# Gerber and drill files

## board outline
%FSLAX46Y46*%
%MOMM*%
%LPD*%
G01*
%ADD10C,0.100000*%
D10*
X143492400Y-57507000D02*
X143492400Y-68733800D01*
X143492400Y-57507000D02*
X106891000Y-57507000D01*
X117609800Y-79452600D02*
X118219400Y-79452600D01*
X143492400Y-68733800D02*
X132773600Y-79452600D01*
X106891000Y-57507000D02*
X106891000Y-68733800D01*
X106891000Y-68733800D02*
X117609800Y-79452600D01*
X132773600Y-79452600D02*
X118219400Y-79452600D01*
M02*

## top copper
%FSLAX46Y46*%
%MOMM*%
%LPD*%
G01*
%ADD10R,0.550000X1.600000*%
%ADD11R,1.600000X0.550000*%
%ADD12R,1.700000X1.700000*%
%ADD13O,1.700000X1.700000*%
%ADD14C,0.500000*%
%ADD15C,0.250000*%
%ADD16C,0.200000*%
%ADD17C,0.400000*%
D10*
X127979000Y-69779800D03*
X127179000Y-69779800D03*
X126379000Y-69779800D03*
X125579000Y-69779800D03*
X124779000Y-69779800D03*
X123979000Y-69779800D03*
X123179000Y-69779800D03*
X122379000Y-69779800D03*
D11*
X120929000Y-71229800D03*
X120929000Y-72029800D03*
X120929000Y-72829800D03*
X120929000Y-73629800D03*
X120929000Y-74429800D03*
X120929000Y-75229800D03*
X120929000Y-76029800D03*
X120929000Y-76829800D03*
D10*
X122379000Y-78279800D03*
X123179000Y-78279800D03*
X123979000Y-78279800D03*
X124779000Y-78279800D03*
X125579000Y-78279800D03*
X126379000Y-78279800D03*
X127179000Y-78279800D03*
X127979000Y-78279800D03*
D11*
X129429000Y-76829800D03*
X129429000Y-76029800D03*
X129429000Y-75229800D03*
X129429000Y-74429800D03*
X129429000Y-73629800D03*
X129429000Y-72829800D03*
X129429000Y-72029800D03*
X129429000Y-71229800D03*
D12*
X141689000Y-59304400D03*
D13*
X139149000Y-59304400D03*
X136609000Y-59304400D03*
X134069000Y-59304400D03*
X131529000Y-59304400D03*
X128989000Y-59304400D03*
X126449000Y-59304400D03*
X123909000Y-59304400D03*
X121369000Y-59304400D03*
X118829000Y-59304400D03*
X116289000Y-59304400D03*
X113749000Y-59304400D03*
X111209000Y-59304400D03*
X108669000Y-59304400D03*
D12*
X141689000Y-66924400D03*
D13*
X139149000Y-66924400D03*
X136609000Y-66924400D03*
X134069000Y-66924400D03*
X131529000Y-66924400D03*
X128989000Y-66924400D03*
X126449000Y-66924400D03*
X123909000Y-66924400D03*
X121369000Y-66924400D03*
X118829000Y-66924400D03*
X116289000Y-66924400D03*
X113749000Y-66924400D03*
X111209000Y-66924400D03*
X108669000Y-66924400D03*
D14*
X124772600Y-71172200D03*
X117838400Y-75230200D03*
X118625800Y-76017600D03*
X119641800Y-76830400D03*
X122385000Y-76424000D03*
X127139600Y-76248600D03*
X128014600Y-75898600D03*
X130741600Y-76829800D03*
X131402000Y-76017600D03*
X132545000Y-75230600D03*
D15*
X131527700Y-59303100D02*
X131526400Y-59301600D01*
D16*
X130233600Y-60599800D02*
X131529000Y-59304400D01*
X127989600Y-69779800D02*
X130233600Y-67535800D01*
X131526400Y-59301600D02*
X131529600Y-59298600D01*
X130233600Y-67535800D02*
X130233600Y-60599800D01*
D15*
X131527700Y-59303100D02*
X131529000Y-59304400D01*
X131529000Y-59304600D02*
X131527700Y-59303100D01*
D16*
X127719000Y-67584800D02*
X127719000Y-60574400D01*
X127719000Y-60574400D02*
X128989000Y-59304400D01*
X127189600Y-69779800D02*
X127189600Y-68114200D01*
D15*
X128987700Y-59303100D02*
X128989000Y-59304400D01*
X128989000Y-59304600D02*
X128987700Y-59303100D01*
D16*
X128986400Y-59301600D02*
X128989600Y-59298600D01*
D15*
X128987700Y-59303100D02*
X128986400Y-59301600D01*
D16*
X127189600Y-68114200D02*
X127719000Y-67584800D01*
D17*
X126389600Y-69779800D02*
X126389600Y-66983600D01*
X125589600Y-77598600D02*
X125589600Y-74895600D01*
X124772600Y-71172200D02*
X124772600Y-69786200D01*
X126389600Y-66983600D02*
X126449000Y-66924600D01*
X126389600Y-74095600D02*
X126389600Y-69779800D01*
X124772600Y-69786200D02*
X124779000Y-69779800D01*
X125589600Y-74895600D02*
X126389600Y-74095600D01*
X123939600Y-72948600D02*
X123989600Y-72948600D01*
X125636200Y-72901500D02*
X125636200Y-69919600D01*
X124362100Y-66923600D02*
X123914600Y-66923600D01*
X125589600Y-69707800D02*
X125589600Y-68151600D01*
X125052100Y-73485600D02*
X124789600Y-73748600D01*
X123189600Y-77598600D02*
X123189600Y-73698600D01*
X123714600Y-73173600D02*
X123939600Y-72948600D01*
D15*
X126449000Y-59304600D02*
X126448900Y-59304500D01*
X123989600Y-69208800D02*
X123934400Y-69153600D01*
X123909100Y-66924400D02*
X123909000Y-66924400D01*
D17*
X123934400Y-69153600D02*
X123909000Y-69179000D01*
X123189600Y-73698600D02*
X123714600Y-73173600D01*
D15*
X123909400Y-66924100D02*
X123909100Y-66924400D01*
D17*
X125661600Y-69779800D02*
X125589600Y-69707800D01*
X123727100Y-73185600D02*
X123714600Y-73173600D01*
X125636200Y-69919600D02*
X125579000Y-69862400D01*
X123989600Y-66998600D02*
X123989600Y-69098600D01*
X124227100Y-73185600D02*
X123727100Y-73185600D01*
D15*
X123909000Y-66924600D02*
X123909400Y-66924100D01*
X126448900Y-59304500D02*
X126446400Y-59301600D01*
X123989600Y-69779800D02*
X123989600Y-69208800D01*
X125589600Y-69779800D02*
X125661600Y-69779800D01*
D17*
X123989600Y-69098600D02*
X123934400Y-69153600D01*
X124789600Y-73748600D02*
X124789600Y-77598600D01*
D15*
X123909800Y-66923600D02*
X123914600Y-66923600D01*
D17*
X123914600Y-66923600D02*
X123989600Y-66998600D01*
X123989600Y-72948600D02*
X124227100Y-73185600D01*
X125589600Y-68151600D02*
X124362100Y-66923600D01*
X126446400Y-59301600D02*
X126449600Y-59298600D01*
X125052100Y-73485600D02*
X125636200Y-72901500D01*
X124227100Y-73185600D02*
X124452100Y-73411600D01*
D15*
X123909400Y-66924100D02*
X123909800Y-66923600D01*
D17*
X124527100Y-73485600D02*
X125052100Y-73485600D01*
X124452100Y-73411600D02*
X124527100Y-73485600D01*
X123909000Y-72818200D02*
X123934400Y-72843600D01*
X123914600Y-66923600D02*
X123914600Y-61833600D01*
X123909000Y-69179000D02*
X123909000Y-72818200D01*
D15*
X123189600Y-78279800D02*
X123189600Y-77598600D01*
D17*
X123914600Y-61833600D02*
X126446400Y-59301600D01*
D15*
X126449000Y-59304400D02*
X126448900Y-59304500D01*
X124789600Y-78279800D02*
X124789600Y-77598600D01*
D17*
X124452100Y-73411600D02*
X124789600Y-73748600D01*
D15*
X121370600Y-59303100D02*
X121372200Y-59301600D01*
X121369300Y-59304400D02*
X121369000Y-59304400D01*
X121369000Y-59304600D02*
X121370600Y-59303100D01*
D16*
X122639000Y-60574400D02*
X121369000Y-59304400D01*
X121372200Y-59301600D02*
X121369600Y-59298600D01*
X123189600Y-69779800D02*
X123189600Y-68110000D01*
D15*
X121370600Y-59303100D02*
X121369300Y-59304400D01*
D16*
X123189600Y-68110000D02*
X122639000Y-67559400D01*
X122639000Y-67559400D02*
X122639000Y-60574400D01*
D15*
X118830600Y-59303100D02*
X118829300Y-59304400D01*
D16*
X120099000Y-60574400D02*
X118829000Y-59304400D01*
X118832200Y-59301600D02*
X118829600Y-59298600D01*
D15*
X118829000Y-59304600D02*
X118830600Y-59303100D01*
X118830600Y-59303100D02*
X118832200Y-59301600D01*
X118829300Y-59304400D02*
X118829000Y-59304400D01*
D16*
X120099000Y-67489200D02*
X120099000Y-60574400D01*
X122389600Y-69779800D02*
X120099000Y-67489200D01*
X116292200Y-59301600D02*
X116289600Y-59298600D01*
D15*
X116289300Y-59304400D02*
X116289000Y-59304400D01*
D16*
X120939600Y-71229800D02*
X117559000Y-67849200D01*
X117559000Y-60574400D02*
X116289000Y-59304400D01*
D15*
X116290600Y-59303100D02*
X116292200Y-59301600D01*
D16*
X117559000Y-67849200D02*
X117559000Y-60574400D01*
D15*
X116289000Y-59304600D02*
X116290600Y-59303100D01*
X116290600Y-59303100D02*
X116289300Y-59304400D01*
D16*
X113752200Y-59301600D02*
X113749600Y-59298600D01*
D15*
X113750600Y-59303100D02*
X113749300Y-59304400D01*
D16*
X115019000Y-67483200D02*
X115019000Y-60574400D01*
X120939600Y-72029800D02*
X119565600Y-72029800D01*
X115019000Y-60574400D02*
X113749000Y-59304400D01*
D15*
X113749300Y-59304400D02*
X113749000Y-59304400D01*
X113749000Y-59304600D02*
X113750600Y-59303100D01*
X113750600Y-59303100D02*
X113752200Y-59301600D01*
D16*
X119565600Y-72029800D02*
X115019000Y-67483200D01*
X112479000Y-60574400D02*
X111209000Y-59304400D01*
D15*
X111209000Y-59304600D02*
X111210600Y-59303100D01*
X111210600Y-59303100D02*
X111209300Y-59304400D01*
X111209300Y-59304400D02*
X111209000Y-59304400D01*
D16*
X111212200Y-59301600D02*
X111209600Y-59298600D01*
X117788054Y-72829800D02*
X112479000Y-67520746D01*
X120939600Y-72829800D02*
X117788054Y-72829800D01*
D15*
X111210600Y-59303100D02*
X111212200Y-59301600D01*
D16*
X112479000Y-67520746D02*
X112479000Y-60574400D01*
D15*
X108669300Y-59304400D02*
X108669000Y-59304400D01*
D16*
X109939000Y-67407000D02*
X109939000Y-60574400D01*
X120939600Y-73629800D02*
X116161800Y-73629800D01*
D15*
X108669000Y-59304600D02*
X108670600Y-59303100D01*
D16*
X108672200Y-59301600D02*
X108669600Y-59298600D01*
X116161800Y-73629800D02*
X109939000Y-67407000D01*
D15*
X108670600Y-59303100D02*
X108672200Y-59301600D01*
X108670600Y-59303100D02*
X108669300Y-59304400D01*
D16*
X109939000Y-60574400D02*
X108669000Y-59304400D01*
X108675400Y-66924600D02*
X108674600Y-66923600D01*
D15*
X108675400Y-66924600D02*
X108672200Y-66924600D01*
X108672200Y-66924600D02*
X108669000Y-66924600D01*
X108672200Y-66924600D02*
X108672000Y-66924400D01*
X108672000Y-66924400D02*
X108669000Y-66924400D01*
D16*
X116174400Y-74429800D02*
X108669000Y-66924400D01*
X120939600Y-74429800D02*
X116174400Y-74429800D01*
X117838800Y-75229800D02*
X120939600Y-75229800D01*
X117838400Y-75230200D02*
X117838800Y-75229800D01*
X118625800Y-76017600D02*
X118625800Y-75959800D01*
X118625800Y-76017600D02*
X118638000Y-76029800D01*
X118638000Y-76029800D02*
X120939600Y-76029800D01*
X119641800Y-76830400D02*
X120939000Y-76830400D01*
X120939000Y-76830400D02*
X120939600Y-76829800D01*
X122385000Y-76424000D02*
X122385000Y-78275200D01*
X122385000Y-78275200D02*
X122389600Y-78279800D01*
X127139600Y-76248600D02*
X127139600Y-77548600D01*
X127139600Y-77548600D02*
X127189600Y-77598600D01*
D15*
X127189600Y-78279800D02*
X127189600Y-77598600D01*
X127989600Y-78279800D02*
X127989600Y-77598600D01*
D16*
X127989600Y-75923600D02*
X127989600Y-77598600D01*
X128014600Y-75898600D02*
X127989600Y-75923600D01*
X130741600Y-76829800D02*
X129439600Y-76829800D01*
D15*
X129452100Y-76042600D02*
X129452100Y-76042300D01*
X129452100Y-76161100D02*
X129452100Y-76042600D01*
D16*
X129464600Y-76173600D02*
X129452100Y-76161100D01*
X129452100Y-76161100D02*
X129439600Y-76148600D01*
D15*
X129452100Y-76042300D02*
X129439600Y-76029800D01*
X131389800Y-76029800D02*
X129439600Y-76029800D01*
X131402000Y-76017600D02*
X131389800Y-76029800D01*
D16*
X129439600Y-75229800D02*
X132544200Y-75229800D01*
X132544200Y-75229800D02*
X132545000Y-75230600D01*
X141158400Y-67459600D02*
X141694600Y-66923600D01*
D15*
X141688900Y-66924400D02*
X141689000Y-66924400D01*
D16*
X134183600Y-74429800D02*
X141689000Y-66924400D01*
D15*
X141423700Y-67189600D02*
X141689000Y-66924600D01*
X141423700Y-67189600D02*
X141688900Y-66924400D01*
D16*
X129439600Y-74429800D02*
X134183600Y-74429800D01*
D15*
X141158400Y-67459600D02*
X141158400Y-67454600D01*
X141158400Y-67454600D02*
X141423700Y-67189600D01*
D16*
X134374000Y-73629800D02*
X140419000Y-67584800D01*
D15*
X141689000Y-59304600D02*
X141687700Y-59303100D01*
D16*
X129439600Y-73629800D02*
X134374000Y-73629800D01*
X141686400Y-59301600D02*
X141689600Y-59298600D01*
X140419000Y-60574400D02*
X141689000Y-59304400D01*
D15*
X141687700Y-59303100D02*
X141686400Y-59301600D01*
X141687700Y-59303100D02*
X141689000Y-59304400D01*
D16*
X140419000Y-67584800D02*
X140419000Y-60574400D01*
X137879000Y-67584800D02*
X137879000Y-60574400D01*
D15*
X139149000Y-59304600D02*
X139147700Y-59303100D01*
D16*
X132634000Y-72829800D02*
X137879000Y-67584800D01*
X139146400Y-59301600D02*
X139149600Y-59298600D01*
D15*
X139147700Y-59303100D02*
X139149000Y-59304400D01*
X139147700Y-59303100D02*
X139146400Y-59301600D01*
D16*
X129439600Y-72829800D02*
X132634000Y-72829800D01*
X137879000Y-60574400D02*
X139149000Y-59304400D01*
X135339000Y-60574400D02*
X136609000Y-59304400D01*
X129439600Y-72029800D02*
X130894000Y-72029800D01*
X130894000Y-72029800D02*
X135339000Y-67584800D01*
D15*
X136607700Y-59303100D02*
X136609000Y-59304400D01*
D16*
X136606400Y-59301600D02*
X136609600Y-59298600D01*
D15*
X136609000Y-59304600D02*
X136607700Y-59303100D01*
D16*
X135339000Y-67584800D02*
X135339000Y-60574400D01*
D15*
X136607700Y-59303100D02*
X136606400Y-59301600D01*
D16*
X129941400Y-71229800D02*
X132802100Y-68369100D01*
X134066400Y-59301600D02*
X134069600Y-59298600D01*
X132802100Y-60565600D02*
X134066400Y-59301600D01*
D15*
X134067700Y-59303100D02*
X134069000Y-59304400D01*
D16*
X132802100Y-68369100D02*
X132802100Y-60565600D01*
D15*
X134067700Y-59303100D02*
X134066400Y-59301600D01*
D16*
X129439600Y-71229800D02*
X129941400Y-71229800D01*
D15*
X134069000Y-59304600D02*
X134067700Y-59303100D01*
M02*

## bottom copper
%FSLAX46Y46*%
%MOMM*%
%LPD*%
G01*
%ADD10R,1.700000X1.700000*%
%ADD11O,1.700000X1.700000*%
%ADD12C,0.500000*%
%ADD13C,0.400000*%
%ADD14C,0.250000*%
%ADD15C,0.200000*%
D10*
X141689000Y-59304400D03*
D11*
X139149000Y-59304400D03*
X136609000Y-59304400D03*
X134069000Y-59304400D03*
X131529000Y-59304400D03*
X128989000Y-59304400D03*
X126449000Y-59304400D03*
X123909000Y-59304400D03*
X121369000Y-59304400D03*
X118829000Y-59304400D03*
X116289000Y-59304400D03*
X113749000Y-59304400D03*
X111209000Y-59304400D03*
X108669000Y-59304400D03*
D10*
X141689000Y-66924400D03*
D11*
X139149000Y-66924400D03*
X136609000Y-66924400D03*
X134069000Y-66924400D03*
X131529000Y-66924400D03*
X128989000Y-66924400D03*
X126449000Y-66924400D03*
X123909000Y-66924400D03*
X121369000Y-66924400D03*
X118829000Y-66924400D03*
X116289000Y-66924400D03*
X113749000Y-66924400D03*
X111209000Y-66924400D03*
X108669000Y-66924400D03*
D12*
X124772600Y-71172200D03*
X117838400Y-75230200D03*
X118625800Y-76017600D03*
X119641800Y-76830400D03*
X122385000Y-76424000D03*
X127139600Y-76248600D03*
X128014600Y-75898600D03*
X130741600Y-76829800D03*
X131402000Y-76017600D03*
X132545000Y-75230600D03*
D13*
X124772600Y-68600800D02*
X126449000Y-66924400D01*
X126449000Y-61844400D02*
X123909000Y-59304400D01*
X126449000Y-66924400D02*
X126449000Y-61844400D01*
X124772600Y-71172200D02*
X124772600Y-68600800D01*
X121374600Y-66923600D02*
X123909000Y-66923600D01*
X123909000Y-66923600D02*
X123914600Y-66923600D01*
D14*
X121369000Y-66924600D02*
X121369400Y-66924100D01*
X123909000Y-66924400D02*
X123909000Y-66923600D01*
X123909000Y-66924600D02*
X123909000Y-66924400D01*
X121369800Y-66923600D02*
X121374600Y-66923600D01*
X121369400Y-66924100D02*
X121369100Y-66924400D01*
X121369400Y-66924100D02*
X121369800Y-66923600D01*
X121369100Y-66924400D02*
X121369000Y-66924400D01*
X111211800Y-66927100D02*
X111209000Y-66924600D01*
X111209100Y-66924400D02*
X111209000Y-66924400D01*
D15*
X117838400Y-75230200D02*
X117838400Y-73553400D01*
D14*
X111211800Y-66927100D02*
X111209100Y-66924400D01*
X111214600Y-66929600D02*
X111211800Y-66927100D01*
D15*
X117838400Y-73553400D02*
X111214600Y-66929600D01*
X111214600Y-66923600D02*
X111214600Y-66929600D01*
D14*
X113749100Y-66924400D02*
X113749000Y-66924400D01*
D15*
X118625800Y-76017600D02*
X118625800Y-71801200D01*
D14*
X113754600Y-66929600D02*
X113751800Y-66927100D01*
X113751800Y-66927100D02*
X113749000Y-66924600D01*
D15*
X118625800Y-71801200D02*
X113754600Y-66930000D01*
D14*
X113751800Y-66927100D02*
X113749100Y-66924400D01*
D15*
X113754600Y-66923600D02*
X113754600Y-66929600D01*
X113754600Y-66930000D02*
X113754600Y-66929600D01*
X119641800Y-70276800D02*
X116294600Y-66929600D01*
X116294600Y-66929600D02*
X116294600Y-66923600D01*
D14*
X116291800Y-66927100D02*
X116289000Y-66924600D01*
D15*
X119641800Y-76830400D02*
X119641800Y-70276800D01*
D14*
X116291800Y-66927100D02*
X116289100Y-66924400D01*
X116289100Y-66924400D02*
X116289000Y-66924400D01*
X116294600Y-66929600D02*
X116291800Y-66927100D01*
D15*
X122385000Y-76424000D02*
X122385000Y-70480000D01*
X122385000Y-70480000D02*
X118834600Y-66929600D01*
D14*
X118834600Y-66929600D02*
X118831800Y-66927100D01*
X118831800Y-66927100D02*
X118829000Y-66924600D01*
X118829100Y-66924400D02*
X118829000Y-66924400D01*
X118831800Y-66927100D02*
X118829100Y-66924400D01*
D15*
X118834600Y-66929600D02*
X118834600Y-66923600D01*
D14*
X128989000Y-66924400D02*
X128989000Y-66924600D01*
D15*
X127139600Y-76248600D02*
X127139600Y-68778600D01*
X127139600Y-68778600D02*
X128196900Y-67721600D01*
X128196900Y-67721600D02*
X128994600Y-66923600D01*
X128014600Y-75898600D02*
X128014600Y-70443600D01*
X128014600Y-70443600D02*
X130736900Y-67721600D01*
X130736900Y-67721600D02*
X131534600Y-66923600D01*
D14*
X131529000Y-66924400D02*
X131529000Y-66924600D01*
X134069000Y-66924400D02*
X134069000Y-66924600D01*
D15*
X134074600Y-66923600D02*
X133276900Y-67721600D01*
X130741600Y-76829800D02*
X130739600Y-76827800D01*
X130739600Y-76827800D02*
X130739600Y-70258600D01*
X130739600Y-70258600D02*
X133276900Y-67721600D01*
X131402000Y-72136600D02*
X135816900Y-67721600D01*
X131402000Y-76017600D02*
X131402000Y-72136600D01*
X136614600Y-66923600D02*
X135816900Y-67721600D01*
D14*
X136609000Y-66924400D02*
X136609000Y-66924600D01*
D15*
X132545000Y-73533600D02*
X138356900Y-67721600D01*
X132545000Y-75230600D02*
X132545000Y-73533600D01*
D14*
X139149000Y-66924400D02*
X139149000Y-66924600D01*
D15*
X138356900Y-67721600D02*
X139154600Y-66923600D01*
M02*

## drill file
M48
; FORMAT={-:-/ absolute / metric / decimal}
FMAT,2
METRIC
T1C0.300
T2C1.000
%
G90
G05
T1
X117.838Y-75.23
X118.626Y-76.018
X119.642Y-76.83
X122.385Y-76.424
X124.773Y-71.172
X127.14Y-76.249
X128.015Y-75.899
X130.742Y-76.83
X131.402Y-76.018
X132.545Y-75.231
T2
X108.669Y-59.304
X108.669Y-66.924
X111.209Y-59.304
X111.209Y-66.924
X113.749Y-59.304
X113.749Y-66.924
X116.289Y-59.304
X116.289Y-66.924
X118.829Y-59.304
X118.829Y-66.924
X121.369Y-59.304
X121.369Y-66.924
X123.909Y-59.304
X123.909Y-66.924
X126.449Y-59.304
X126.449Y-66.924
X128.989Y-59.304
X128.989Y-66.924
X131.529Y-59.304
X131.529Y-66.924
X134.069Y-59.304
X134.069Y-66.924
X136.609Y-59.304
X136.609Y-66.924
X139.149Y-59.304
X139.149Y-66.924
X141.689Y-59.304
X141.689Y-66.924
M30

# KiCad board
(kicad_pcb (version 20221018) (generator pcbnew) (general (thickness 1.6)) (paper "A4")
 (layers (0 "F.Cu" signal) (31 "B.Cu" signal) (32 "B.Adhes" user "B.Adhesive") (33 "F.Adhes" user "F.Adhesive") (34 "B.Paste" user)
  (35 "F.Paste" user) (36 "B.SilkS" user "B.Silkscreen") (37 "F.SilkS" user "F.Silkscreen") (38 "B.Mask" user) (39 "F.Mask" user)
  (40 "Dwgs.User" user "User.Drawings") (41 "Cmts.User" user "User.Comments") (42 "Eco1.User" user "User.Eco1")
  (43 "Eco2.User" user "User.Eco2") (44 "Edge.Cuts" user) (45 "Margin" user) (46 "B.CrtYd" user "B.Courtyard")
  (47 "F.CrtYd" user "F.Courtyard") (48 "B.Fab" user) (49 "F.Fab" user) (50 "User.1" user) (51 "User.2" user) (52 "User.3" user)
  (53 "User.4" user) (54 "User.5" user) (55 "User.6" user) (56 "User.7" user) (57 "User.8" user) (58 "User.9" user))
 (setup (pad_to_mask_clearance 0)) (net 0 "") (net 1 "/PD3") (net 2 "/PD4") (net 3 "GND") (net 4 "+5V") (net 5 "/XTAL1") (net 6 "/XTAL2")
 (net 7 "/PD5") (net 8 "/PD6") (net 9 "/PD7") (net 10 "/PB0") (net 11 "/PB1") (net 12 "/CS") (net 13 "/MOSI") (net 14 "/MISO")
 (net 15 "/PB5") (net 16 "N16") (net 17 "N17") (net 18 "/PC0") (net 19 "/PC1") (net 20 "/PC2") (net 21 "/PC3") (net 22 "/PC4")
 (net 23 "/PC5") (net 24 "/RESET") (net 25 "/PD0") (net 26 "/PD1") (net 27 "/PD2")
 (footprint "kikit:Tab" (layer "F.Cu") (at 113.0505 57.277 -90)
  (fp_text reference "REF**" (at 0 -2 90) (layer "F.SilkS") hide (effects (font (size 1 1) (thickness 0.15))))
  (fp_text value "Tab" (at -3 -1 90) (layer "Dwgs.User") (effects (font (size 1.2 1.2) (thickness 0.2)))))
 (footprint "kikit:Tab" (layer "F.Cu") (at 125.4965 79.7052 90)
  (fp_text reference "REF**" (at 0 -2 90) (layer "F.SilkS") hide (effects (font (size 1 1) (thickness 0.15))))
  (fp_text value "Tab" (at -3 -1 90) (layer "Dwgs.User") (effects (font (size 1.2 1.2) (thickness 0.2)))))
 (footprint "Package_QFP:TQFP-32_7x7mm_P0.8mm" (layer "F.Cu") (at 125.179 74.0298 -90)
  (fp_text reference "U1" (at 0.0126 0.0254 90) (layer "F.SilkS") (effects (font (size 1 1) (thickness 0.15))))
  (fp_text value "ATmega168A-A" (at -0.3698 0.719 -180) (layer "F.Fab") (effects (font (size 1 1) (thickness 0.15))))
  (pad "1" smd rect (at -4.25 -2.8 270) (size 1.6 0.55) (layers "F.Cu" "F.Paste" "F.Mask") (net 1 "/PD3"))
  (pad "2" smd rect (at -4.25 -2 270) (size 1.6 0.55) (layers "F.Cu" "F.Paste" "F.Mask") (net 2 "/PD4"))
  (pad "3" smd rect (at -4.25 -1.2 270) (size 1.6 0.55) (layers "F.Cu" "F.Paste" "F.Mask") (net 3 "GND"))
  (pad "4" smd rect (at -4.25 -0.4 270) (size 1.6 0.55) (layers "F.Cu" "F.Paste" "F.Mask") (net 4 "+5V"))
  (pad "5" smd rect (at -4.25 0.4 270) (size 1.6 0.55) (layers "F.Cu" "F.Paste" "F.Mask") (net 3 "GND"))
  (pad "6" smd rect (at -4.25 1.2 270) (size 1.6 0.55) (layers "F.Cu" "F.Paste" "F.Mask") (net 4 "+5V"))
  (pad "7" smd rect (at -4.25 2 270) (size 1.6 0.55) (layers "F.Cu" "F.Paste" "F.Mask") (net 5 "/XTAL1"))
  (pad "8" smd rect (at -4.25 2.8 270) (size 1.6 0.55) (layers "F.Cu" "F.Paste" "F.Mask") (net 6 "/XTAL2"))
  (pad "9" smd rect (at -2.8 4.25) (size 1.6 0.55) (layers "F.Cu" "F.Paste" "F.Mask") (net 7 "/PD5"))
  (pad "10" smd rect (at -2 4.25) (size 1.6 0.55) (layers "F.Cu" "F.Paste" "F.Mask") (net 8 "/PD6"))
  (pad "11" smd rect (at -1.2 4.25) (size 1.6 0.55) (layers "F.Cu" "F.Paste" "F.Mask") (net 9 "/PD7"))
  (pad "12" smd rect (at -0.4 4.25) (size 1.6 0.55) (layers "F.Cu" "F.Paste" "F.Mask") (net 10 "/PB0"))
  (pad "13" smd rect (at 0.4 4.25) (size 1.6 0.55) (layers "F.Cu" "F.Paste" "F.Mask") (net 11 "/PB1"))
  (pad "14" smd rect (at 1.2 4.25) (size 1.6 0.55) (layers "F.Cu" "F.Paste" "F.Mask") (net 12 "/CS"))
  (pad "15" smd rect (at 2 4.25) (size 1.6 0.55) (layers "F.Cu" "F.Paste" "F.Mask") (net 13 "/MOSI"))
  (pad "16" smd rect (at 2.8 4.25) (size 1.6 0.55) (layers "F.Cu" "F.Paste" "F.Mask") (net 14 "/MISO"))
  (pad "17" smd rect (at 4.25 2.8 270) (size 1.6 0.55) (layers "F.Cu" "F.Paste" "F.Mask") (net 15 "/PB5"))
  (pad "18" smd rect (at 4.25 2 270) (size 1.6 0.55) (layers "F.Cu" "F.Paste" "F.Mask") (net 4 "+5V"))
  (pad "19" smd rect (at 4.25 1.2 270) (size 1.6 0.55) (layers "F.Cu" "F.Paste" "F.Mask") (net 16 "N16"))
  (pad "20" smd rect (at 4.25 0.4 270) (size 1.6 0.55) (layers "F.Cu" "F.Paste" "F.Mask") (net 4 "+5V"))
  (pad "21" smd rect (at 4.25 -0.4 270) (size 1.6 0.55) (layers "F.Cu" "F.Paste" "F.Mask") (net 3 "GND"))
  (pad "22" smd rect (at 4.25 -1.2 270) (size 1.6 0.55) (layers "F.Cu" "F.Paste" "F.Mask") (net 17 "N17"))
  (pad "23" smd rect (at 4.25 -2 270) (size 1.6 0.55) (layers "F.Cu" "F.Paste" "F.Mask") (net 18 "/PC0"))
  (pad "24" smd rect (at 4.25 -2.8 270) (size 1.6 0.55) (layers "F.Cu" "F.Paste" "F.Mask") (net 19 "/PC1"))
  (pad "25" smd rect (at 2.8 -4.25) (size 1.6 0.55) (layers "F.Cu" "F.Paste" "F.Mask") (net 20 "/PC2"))
  (pad "26" smd rect (at 2 -4.25) (size 1.6 0.55) (layers "F.Cu" "F.Paste" "F.Mask") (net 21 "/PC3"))
  (pad "27" smd rect (at 1.2 -4.25) (size 1.6 0.55) (layers "F.Cu" "F.Paste" "F.Mask") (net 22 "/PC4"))
  (pad "28" smd rect (at 0.4 -4.25) (size 1.6 0.55) (layers "F.Cu" "F.Paste" "F.Mask") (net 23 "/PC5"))
  (pad "29" smd rect (at -0.4 -4.25) (size 1.6 0.55) (layers "F.Cu" "F.Paste" "F.Mask") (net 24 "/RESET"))
  (pad "30" smd rect (at -1.2 -4.25) (size 1.6 0.55) (layers "F.Cu" "F.Paste" "F.Mask") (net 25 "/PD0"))
  (pad "31" smd rect (at -2 -4.25) (size 1.6 0.55) (layers "F.Cu" "F.Paste" "F.Mask") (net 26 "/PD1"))
  (pad "32" smd rect (at -2.8 -4.25) (size 1.6 0.55) (layers "F.Cu" "F.Paste" "F.Mask") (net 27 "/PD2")))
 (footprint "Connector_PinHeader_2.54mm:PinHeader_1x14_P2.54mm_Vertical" (layer "F.Cu") (at 141.689 59.3044 -90)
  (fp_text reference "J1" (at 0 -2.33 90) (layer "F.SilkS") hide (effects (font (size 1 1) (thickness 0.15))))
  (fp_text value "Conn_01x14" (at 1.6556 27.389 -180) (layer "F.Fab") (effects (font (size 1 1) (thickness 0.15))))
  (pad "1" thru_hole rect (at 0 0 270) (size 1.7 1.7) (drill 1) (layers "*.Cu" "*.Mask") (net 24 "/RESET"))
  (pad "2" thru_hole oval (at 0 2.54 270) (size 1.7 1.7) (drill 1) (layers "*.Cu" "*.Mask") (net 25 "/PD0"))
  (pad "3" thru_hole oval (at 0 5.08 270) (size 1.7 1.7) (drill 1) (layers "*.Cu" "*.Mask") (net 26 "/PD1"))
  (pad "4" thru_hole oval (at 0 7.62 270) (size 1.7 1.7) (drill 1) (layers "*.Cu" "*.Mask") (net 27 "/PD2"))
  (pad "5" thru_hole oval (at 0 10.16 270) (size 1.7 1.7) (drill 1) (layers "*.Cu" "*.Mask") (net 1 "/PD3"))
  (pad "6" thru_hole oval (at 0 12.7 270) (size 1.7 1.7) (drill 1) (layers "*.Cu" "*.Mask") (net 2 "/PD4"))
  (pad "7" thru_hole oval (at 0 15.24 270) (size 1.7 1.7) (drill 1) (layers "*.Cu" "*.Mask") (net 4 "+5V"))
  (pad "8" thru_hole oval (at 0 17.78 270) (size 1.7 1.7) (drill 1) (layers "*.Cu" "*.Mask") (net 3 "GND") (zone_connect 2))
  (pad "9" thru_hole oval (at 0 20.32 270) (size 1.7 1.7) (drill 1) (layers "*.Cu" "*.Mask") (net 5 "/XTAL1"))
  (pad "10" thru_hole oval (at 0 22.86 270) (size 1.7 1.7) (drill 1) (layers "*.Cu" "*.Mask") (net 6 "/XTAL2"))
  (pad "11" thru_hole oval (at 0 25.4 270) (size 1.7 1.7) (drill 1) (layers "*.Cu" "*.Mask") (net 7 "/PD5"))
  (pad "12" thru_hole oval (at 0 27.94 270) (size 1.7 1.7) (drill 1) (layers "*.Cu" "*.Mask") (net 8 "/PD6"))
  (pad "13" thru_hole oval (at 0 30.48 270) (size 1.7 1.7) (drill 1) (layers "*.Cu" "*.Mask") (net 9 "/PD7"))
  (pad "14" thru_hole oval (at 0 33.02 270) (size 1.7 1.7) (drill 1) (layers "*.Cu" "*.Mask") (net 10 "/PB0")))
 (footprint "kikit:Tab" (layer "F.Cu") (at 143.7386 63.1204 180)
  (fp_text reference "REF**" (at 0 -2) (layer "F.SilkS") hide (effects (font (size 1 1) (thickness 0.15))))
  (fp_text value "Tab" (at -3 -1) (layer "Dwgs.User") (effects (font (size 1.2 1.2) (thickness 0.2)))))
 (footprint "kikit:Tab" (layer "F.Cu") (at 137.3329 57.2262 -90)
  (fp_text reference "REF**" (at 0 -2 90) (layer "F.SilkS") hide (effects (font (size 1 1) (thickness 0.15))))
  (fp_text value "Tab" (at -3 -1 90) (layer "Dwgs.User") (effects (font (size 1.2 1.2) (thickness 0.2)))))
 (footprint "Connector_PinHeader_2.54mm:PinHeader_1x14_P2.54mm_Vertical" (layer "F.Cu") (at 141.689 66.9244 -90)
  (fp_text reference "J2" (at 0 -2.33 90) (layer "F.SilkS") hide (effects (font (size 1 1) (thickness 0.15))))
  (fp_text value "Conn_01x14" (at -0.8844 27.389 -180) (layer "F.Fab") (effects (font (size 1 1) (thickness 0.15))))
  (pad "1" thru_hole rect (at 0 0 270) (size 1.7 1.7) (drill 1) (layers "*.Cu" "*.Mask") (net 23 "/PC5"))
  (pad "2" thru_hole oval (at 0 2.54 270) (size 1.7 1.7) (drill 1) (layers "*.Cu" "*.Mask") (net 22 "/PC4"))
  (pad "3" thru_hole oval (at 0 5.08 270) (size 1.7 1.7) (drill 1) (layers "*.Cu" "*.Mask") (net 21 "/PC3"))
  (pad "4" thru_hole oval (at 0 7.62 270) (size 1.7 1.7) (drill 1) (layers "*.Cu" "*.Mask") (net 20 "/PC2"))
  (pad "5" thru_hole oval (at 0 10.16 270) (size 1.7 1.7) (drill 1) (layers "*.Cu" "*.Mask") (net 19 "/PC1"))
  (pad "6" thru_hole oval (at 0 12.7 270) (size 1.7 1.7) (drill 1) (layers "*.Cu" "*.Mask") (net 18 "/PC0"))
  (pad "7" thru_hole oval (at 0 15.24 270) (size 1.7 1.7) (drill 1) (layers "*.Cu" "*.Mask") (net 3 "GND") (zone_connect 2))
  (pad "8" thru_hole oval (at 0 17.78 270) (size 1.7 1.7) (drill 1) (layers "*.Cu" "*.Mask") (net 4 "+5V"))
  (pad "9" thru_hole oval (at 0 20.32 270) (size 1.7 1.7) (drill 1) (layers "*.Cu" "*.Mask") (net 4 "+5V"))
  (pad "10" thru_hole oval (at 0 22.86 270) (size 1.7 1.7) (drill 1) (layers "*.Cu" "*.Mask") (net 15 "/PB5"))
  (pad "11" thru_hole oval (at 0 25.4 270) (size 1.7 1.7) (drill 1) (layers "*.Cu" "*.Mask") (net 14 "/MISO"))
  (pad "12" thru_hole oval (at 0 27.94 270) (size 1.7 1.7) (drill 1) (layers "*.Cu" "*.Mask") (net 13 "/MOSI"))
  (pad "13" thru_hole oval (at 0 30.48 270) (size 1.7 1.7) (drill 1) (layers "*.Cu" "*.Mask") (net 12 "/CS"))
  (pad "14" thru_hole oval (at 0 33.02 270) (size 1.7 1.7) (drill 1) (layers "*.Cu" "*.Mask") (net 11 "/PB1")))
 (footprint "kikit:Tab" (layer "F.Cu") (at 106.6292 63.1204)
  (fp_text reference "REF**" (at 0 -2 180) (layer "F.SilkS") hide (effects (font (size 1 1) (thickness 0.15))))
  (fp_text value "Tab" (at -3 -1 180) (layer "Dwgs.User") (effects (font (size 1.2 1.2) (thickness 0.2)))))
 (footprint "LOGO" (layer "B.Cu") (at 125.179 74.0298 180)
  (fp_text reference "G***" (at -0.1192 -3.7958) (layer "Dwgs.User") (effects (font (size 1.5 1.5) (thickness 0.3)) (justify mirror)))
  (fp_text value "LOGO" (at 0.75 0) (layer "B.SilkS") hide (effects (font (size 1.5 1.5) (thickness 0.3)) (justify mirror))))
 (gr_line (start 143.4924 57.507) (end 143.4924 68.7338) (stroke (width 0.1) (type default)) (layer "Edge.Cuts"))
 (gr_line (start 143.4924 57.507) (end 106.891 57.507) (stroke (width 0.1) (type default)) (layer "Edge.Cuts"))
 (gr_line (start 117.6098 79.4526) (end 118.2194 79.4526) (stroke (width 0.1) (type default)) (layer "Edge.Cuts"))
 (gr_line (start 143.4924 68.7338) (end 132.7736 79.4526) (stroke (width 0.1) (type default)) (layer "Edge.Cuts"))
 (gr_line (start 106.891 57.507) (end 106.891 68.7338) (stroke (width 0.1) (type default)) (layer "Edge.Cuts"))
 (gr_line (start 106.891 68.7338) (end 117.6098 79.4526) (stroke (width 0.1) (type default)) (layer "Edge.Cuts"))
 (gr_line (start 132.7736 79.4526) (end 118.2194 79.4526) (stroke (width 0.1) (type default)) (layer "Edge.Cuts"))
 (segment (start 131.5277 59.3031) (end 131.5264 59.3016) (width 0.25) (layer "F.Cu") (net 1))
 (segment (start 130.2336 60.5998) (end 131.529 59.3044) (width 0.2) (layer "F.Cu") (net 1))
 (segment (start 127.9896 69.7798) (end 130.2336 67.5358) (width 0.2) (layer "F.Cu") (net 1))
 (segment (start 131.5264 59.3016) (end 131.5296 59.2986) (width 0.2) (layer "F.Cu") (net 1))
 (segment (start 130.2336 67.5358) (end 130.2336 60.5998) (width 0.2) (layer "F.Cu") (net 1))
 (segment (start 131.5277 59.3031) (end 131.529 59.3044) (width 0.25) (layer "F.Cu") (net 1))
 (segment (start 131.529 59.3046) (end 131.5277 59.3031) (width 0.25) (layer "F.Cu") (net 1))
 (segment (start 127.719 67.5848) (end 127.719 60.5744) (width 0.2) (layer "F.Cu") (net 2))
 (segment (start 127.719 60.5744) (end 128.989 59.3044) (width 0.2) (layer "F.Cu") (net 2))
 (segment (start 127.1896 69.7798) (end 127.1896 68.1142) (width 0.2) (layer "F.Cu") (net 2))
 (segment (start 128.9877 59.3031) (end 128.989 59.3044) (width 0.25) (layer "F.Cu") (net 2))
 (segment (start 128.989 59.3046) (end 128.9877 59.3031) (width 0.25) (layer "F.Cu") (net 2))
 (segment (start 128.9864 59.3016) (end 128.9896 59.2986) (width 0.2) (layer "F.Cu") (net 2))
 (segment (start 128.9877 59.3031) (end 128.9864 59.3016) (width 0.25) (layer "F.Cu") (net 2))
 (segment (start 127.1896 68.1142) (end 127.719 67.5848) (width 0.2) (layer "F.Cu") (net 2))
 (segment (start 126.3896 69.7798) (end 126.3896 66.9836) (width 0.4) (layer "F.Cu") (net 3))
 (segment (start 125.5896 77.5986) (end 125.5896 74.8956) (width 0.4) (layer "F.Cu") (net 3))
 (segment (start 124.7726 71.1722) (end 124.7726 69.7862) (width 0.4) (layer "F.Cu") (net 3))
 (segment (start 126.3896 66.9836) (end 126.449 66.9246) (width 0.4) (layer "F.Cu") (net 3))
 (segment (start 126.3896 74.0956) (end 126.3896 69.7798) (width 0.4) (layer "F.Cu") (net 3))
 (segment (start 124.7726 69.7862) (end 124.779 69.7798) (width 0.4) (layer "F.Cu") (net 3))
 (segment (start 125.5896 74.8956) (end 126.3896 74.0956) (width 0.4) (layer "F.Cu") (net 3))
 (via (at 124.7726 71.1722) (size 0.5) (drill 0.3) (layers "F.Cu" "B.Cu") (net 3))
 (segment (start 124.7726 68.6008) (end 126.449 66.9244) (width 0.4) (layer "B.Cu") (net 3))
 (segment (start 126.449 61.8444) (end 123.909 59.3044) (width 0.4) (layer "B.Cu") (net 3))
 (segment (start 126.449 66.9244) (end 126.449 61.8444) (width 0.4) (layer "B.Cu") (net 3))
 (segment (start 124.7726 71.1722) (end 124.7726 68.6008) (width 0.4) (layer "B.Cu") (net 3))
 (segment (start 123.9396 72.9486) (end 123.9896 72.9486) (width 0.4) (layer "F.Cu") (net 4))
 (segment (start 125.6362 72.9015) (end 125.6362 69.9196) (width 0.4) (layer "F.Cu") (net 4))
 (segment (start 124.3621 66.9236) (end 123.9146 66.9236) (width 0.4) (layer "F.Cu") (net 4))
 (segment (start 125.5896 69.7078) (end 125.5896 68.1516) (width 0.4) (layer "F.Cu") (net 4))
 (segment (start 125.0521 73.4856) (end 124.7896 73.7486) (width 0.4) (layer "F.Cu") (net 4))
 (segment (start 123.1896 77.5986) (end 123.1896 73.6986) (width 0.4) (layer "F.Cu") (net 4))
 (segment (start 123.7146 73.1736) (end 123.9396 72.9486) (width 0.4) (layer "F.Cu") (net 4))
 (segment (start 126.449 59.3046) (end 126.4489 59.3045) (width 0.25) (layer "F.Cu") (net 4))
 (segment (start 123.9896 69.2088) (end 123.9344 69.1536) (width 0.25) (layer "F.Cu") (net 4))
 (segment (start 123.9091 66.9244) (end 123.909 66.9244) (width 0.25) (layer "F.Cu") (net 4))
 (segment (start 123.9344 69.1536) (end 123.909 69.179) (width 0.4) (layer "F.Cu") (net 4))
 (segment (start 123.1896 73.6986) (end 123.7146 73.1736) (width 0.4) (layer "F.Cu") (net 4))
 (segment (start 123.9094 66.9241) (end 123.9091 66.9244) (width 0.25) (layer "F.Cu") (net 4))
 (segment (start 125.6616 69.7798) (end 125.5896 69.7078) (width 0.4) (layer "F.Cu") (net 4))
 (segment (start 123.7271 73.1856) (end 123.7146 73.1736) (width 0.4) (layer "F.Cu") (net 4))
 (segment (start 125.6362 69.9196) (end 125.579 69.8624) (width 0.4) (layer "F.Cu") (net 4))
 (segment (start 123.9896 66.9986) (end 123.9896 69.0986) (width 0.4) (layer "F.Cu") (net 4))
 (segment (start 124.2271 73.1856) (end 123.7271 73.1856) (width 0.4) (layer "F.Cu") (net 4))
 (segment (start 123.909 66.9246) (end 123.9094 66.9241) (width 0.25) (layer "F.Cu") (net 4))
 (segment (start 126.4489 59.3045) (end 126.4464 59.3016) (width 0.25) (layer "F.Cu") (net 4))
 (segment (start 123.9896 69.7798) (end 123.9896 69.2088) (width 0.25) (layer "F.Cu") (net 4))
 (segment (start 125.5896 69.7798) (end 125.6616 69.7798) (width 0.25) (layer "F.Cu") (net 4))
 (segment (start 123.9896 69.0986) (end 123.9344 69.1536) (width 0.4) (layer "F.Cu") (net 4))
 (segment (start 124.7896 73.7486) (end 124.7896 77.5986) (width 0.4) (layer "F.Cu") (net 4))
 (segment (start 123.9098 66.9236) (end 123.9146 66.9236) (width 0.25) (layer "F.Cu") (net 4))
 (segment (start 123.9146 66.9236) (end 123.9896 66.9986) (width 0.4) (layer "F.Cu") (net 4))
 (segment (start 123.9896 72.9486) (end 124.2271 73.1856) (width 0.4) (layer "F.Cu") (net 4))
 (segment (start 125.5896 68.1516) (end 124.3621 66.9236) (width 0.4) (layer "F.Cu") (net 4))
 (segment (start 126.4464 59.3016) (end 126.4496 59.2986) (width 0.4) (layer "F.Cu") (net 4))
 (segment (start 125.0521 73.4856) (end 125.6362 72.9015) (width 0.4) (layer "F.Cu") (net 4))
 (segment (start 124.2271 73.1856) (end 124.4521 73.4116) (width 0.4) (layer "F.Cu") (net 4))
 (segment (start 123.9094 66.9241) (end 123.9098 66.9236) (width 0.25) (layer "F.Cu") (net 4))
 (segment (start 124.5271 73.4856) (end 125.0521 73.4856) (width 0.4) (layer "F.Cu") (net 4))
 (segment (start 124.4521 73.4116) (end 124.5271 73.4856) (width 0.4) (layer "F.Cu") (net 4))
 (segment (start 123.909 72.8182) (end 123.9344 72.8436) (width 0.4) (layer "F.Cu") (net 4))
 (segment (start 123.9146 66.9236) (end 123.9146 61.8336) (width 0.4) (layer "F.Cu") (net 4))
 (segment (start 123.909 69.179) (end 123.909 72.8182) (width 0.4) (layer "F.Cu") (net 4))
 (segment (start 123.1896 78.2798) (end 123.1896 77.5986) (width 0.25) (layer "F.Cu") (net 4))
 (segment (start 123.9146 61.8336) (end 126.4464 59.3016) (width 0.4) (layer "F.Cu") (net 4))
 (segment (start 126.449 59.3044) (end 126.4489 59.3045) (width 0.25) (layer "F.Cu") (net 4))
 (segment (start 124.7896 78.2798) (end 124.7896 77.5986) (width 0.25) (layer "F.Cu") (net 4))
 (segment (start 124.4521 73.4116) (end 124.7896 73.7486) (width 0.4) (layer "F.Cu") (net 4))
 (segment (start 121.3746 66.9236) (end 123.909 66.9236) (width 0.4) (layer "B.Cu") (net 4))
 (segment (start 123.909 66.9236) (end 123.9146 66.9236) (width 0.4) (layer "B.Cu") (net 4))
 (segment (start 121.369 66.9246) (end 121.3694 66.9241) (width 0.25) (layer "B.Cu") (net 4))
 (segment (start 123.909 66.9244) (end 123.909 66.9236) (width 0.25) (layer "B.Cu") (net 4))
 (segment (start 123.909 66.9246) (end 123.909 66.9244) (width 0.25) (layer "B.Cu") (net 4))
 (segment (start 121.3698 66.9236) (end 121.3746 66.9236) (width 0.25) (layer "B.Cu") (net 4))
 (segment (start 121.3694 66.9241) (end 121.3691 66.9244) (width 0.25) (layer "B.Cu") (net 4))
 (segment (start 121.3694 66.9241) (end 121.3698 66.9236) (width 0.25) (layer "B.Cu") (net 4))
 (segment (start 121.3691 66.9244) (end 121.369 66.9244) (width 0.25) (layer "B.Cu") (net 4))
 (segment (start 121.3706 59.3031) (end 121.3722 59.3016) (width 0.25) (layer "F.Cu") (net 5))
 (segment (start 121.3693 59.3044) (end 121.369 59.3044) (width 0.25) (layer "F.Cu") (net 5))
 (segment (start 121.369 59.3046) (end 121.3706 59.3031) (width 0.25) (layer "F.Cu") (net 5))
 (segment (start 122.639 60.5744) (end 121.369 59.3044) (width 0.2) (layer "F.Cu") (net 5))
 (segment (start 121.3722 59.3016) (end 121.3696 59.2986) (width 0.2) (layer "F.Cu") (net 5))
 (segment (start 123.1896 69.7798) (end 123.1896 68.11) (width 0.2) (layer "F.Cu") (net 5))
 (segment (start 121.3706 59.3031) (end 121.3693 59.3044) (width 0.25) (layer "F.Cu") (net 5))
 (segment (start 123.1896 68.11) (end 122.639 67.5594) (width 0.2) (layer "F.Cu") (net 5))
 (segment (start 122.639 67.5594) (end 122.639 60.5744) (width 0.2) (layer "F.Cu") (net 5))
 (segment (start 118.8306 59.3031) (end 118.8293 59.3044) (width 0.25) (layer "F.Cu") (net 6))
 (segment (start 120.099 60.5744) (end 118.829 59.3044) (width 0.2) (layer "F.Cu") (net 6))
 (segment (start 118.8322 59.3016) (end 118.8296 59.2986) (width 0.2) (layer "F.Cu") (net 6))
 (segment (start 118.829 59.3046) (end 118.8306 59.3031) (width 0.25) (layer "F.Cu") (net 6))
 (segment (start 118.8306 59.3031) (end 118.8322 59.3016) (width 0.25) (layer "F.Cu") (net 6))
 (segment (start 118.8293 59.3044) (end 118.829 59.3044) (width 0.25) (layer "F.Cu") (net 6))
 (segment (start 120.099 67.4892) (end 120.099 60.5744) (width 0.2) (layer "F.Cu") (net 6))
 (segment (start 122.3896 69.7798) (end 120.099 67.4892) (width 0.2) (layer "F.Cu") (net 6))
 (segment (start 116.2922 59.3016) (end 116.2896 59.2986) (width 0.2) (layer "F.Cu") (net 7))
 (segment (start 116.2893 59.3044) (end 116.289 59.3044) (width 0.25) (layer "F.Cu") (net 7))
 (segment (start 120.9396 71.2298) (end 117.559 67.8492) (width 0.2) (layer "F.Cu") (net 7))
 (segment (start 117.559 60.5744) (end 116.289 59.3044) (width 0.2) (layer "F.Cu") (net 7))
 (segment (start 116.2906 59.3031) (end 116.2922 59.3016) (width 0.25) (layer "F.Cu") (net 7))
 (segment (start 117.559 67.8492) (end 117.559 60.5744) (width 0.2) (layer "F.Cu") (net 7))
 (segment (start 116.289 59.3046) (end 116.2906 59.3031) (width 0.25) (layer "F.Cu") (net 7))
 (segment (start 116.2906 59.3031) (end 116.2893 59.3044) (width 0.25) (layer "F.Cu") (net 7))
 (segment (start 113.7522 59.3016) (end 113.7496 59.2986) (width 0.2) (layer "F.Cu") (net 8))
 (segment (start 113.7506 59.3031) (end 113.7493 59.3044) (width 0.25) (layer "F.Cu") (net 8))
 (segment (start 115.019 67.4832) (end 115.019 60.5744) (width 0.2) (layer "F.Cu") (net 8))
 (segment (start 120.9396 72.0298) (end 119.5656 72.0298) (width 0.2) (layer "F.Cu") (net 8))
 (segment (start 115.019 60.5744) (end 113.749 59.3044) (width 0.2) (layer "F.Cu") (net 8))
 (segment (start 113.7493 59.3044) (end 113.749 59.3044) (width 0.25) (layer "F.Cu") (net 8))
 (segment (start 113.749 59.3046) (end 113.7506 59.3031) (width 0.25) (layer "F.Cu") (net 8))
 (segment (start 113.7506 59.3031) (end 113.7522 59.3016) (width 0.25) (layer "F.Cu") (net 8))
 (segment (start 119.5656 72.0298) (end 115.019 67.4832) (width 0.2) (layer "F.Cu") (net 8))
 (segment (start 112.479 60.5744) (end 111.209 59.3044) (width 0.2) (layer "F.Cu") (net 9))
 (segment (start 111.209 59.3046) (end 111.2106 59.3031) (width 0.25) (layer "F.Cu") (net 9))
 (segment (start 111.2106 59.3031) (end 111.2093 59.3044) (width 0.25) (layer "F.Cu") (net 9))
 (segment (start 111.2093 59.3044) (end 111.209 59.3044) (width 0.25) (layer "F.Cu") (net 9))
 (segment (start 111.2122 59.3016) (end 111.2096 59.2986) (width 0.2) (layer "F.Cu") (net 9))
 (segment (start 117.788054 72.8298) (end 112.479 67.520746) (width 0.2) (layer "F.Cu") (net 9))
 (segment (start 120.9396 72.8298) (end 117.788054 72.8298) (width 0.2) (layer "F.Cu") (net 9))
 (segment (start 111.2106 59.3031) (end 111.2122 59.3016) (width 0.25) (layer "F.Cu") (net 9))
 (segment (start 112.479 67.520746) (end 112.479 60.5744) (width 0.2) (layer "F.Cu") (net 9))
 (segment (start 108.6693 59.3044) (end 108.669 59.3044) (width 0.25) (layer "F.Cu") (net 10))
 (segment (start 109.939 67.407) (end 109.939 60.5744) (width 0.2) (layer "F.Cu") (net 10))
 (segment (start 120.9396 73.6298) (end 116.1618 73.6298) (width 0.2) (layer "F.Cu") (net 10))
 (segment (start 108.669 59.3046) (end 108.6706 59.3031) (width 0.25) (layer "F.Cu") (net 10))
 (segment (start 108.6722 59.3016) (end 108.6696 59.2986) (width 0.2) (layer "F.Cu") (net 10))
 (segment (start 116.1618 73.6298) (end 109.939 67.407) (width 0.2) (layer "F.Cu") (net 10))
 (segment (start 108.6706 59.3031) (end 108.6722 59.3016) (width 0.25) (layer "F.Cu") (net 10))
 (segment (start 108.6706 59.3031) (end 108.6693 59.3044) (width 0.25) (layer "F.Cu") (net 10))
 (segment (start 109.939 60.5744) (end 108.669 59.3044) (width 0.2) (layer "F.Cu") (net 10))
 (segment (start 108.6754 66.9246) (end 108.6746 66.9236) (width 0.2) (layer "F.Cu") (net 11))
 (segment (start 108.6754 66.9246) (end 108.6722 66.9246) (width 0.25) (layer "F.Cu") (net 11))
 (segment (start 108.6722 66.9246) (end 108.669 66.9246) (width 0.25) (layer "F.Cu") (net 11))
 (segment (start 108.6722 66.9246) (end 108.672 66.9244) (width 0.25) (layer "F.Cu") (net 11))
 (segment (start 108.672 66.9244) (end 108.669 66.9244) (width 0.25) (layer "F.Cu") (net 11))
 (segment (start 116.1744 74.4298) (end 108.669 66.9244) (width 0.2) (layer "F.Cu") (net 11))
 (segment (start 120.9396 74.4298) (end 116.1744 74.4298) (width 0.2) (layer "F.Cu") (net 11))
 (segment (start 117.8388 75.2298) (end 120.9396 75.2298) (width 0.2) (layer "F.Cu") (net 12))
 (segment (start 117.8384 75.2302) (end 117.8388 75.2298) (width 0.2) (layer "F.Cu") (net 12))
 (via (at 117.8384 75.2302) (size 0.5) (drill 0.3) (layers "F.Cu" "B.Cu") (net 12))
 (segment (start 111.2118 66.9271) (end 111.209 66.9246) (width 0.25) (layer "B.Cu") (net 12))
 (segment (start 111.2091 66.9244) (end 111.209 66.9244) (width 0.25) (layer "B.Cu") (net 12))
 (segment (start 117.8384 75.2302) (end 117.8384 73.5534) (width 0.2) (layer "B.Cu") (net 12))
 (segment (start 111.2118 66.9271) (end 111.2091 66.9244) (width 0.25) (layer "B.Cu") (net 12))
 (segment (start 111.2146 66.9296) (end 111.2118 66.9271) (width 0.25) (layer "B.Cu") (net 12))
 (segment (start 117.8384 73.5534) (end 111.2146 66.9296) (width 0.2) (layer "B.Cu") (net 12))
 (segment (start 111.2146 66.9236) (end 111.2146 66.9296) (width 0.2) (layer "B.Cu") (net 12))
 (segment (start 118.6258 76.0176) (end 118.6258 75.9598) (width 0.2) (layer "F.Cu") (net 13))
 (segment (start 118.6258 76.0176) (end 118.638 76.0298) (width 0.2) (layer "F.Cu") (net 13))
 (segment (start 118.638 76.0298) (end 120.9396 76.0298) (width 0.2) (layer "F.Cu") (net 13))
 (via (at 118.6258 76.0176) (size 0.5) (drill 0.3) (layers "F.Cu" "B.Cu") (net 13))
 (segment (start 113.7491 66.9244) (end 113.749 66.9244) (width 0.25) (layer "B.Cu") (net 13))
 (segment (start 118.6258 76.0176) (end 118.6258 71.8012) (width 0.2) (layer "B.Cu") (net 13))
 (segment (start 113.7546 66.9296) (end 113.7518 66.9271) (width 0.25) (layer "B.Cu") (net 13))
 (segment (start 113.7518 66.9271) (end 113.749 66.9246) (width 0.25) (layer "B.Cu") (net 13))
 (segment (start 118.6258 71.8012) (end 113.7546 66.93) (width 0.2) (layer "B.Cu") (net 13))
 (segment (start 113.7518 66.9271) (end 113.7491 66.9244) (width 0.25) (layer "B.Cu") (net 13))
 (segment (start 113.7546 66.9236) (end 113.7546 66.9296) (width 0.2) (layer "B.Cu") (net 13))
 (segment (start 113.7546 66.93) (end 113.7546 66.9296) (width 0.2) (layer "B.Cu") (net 13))
 (segment (start 119.6418 76.8304) (end 120.939 76.8304) (width 0.2) (layer "F.Cu") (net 14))
 (segment (start 120.939 76.8304) (end 120.9396 76.8298) (width 0.2) (layer "F.Cu") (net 14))
 (via (at 119.6418 76.8304) (size 0.5) (drill 0.3) (layers "F.Cu" "B.Cu") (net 14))
 (segment (start 119.6418 70.2768) (end 116.2946 66.9296) (width 0.2) (layer "B.Cu") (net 14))
 (segment (start 116.2946 66.9296) (end 116.2946 66.9236) (width 0.2) (layer "B.Cu") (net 14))
 (segment (start 116.2918 66.9271) (end 116.289 66.9246) (width 0.25) (layer "B.Cu") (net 14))
 (segment (start 119.6418 76.8304) (end 119.6418 70.2768) (width 0.2) (layer "B.Cu") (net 14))
 (segment (start 116.2918 66.9271) (end 116.2891 66.9244) (width 0.25) (layer "B.Cu") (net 14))
 (segment (start 116.2891 66.9244) (end 116.289 66.9244) (width 0.25) (layer "B.Cu") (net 14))
 (segment (start 116.2946 66.9296) (end 116.2918 66.9271) (width 0.25) (layer "B.Cu") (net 14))
 (segment (start 122.385 76.424) (end 122.385 78.2752) (width 0.2) (layer "F.Cu") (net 15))
 (segment (start 122.385 78.2752) (end 122.3896 78.2798) (width 0.2) (layer "F.Cu") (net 15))
 (via (at 122.385 76.424) (size 0.5) (drill 0.3) (layers "F.Cu" "B.Cu") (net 15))
 (segment (start 122.385 76.424) (end 122.385 70.48) (width 0.2) (layer "B.Cu") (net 15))
 (segment (start 122.385 70.48) (end 118.8346 66.9296) (width 0.2) (layer "B.Cu") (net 15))
 (segment (start 118.8346 66.9296) (end 118.8318 66.9271) (width 0.25) (layer "B.Cu") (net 15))
 (segment (start 118.8318 66.9271) (end 118.829 66.9246) (width 0.25) (layer "B.Cu") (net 15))
 (segment (start 118.8291 66.9244) (end 118.829 66.9244) (width 0.25) (layer "B.Cu") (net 15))
 (segment (start 118.8318 66.9271) (end 118.8291 66.9244) (width 0.25) (layer "B.Cu") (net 15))
 (segment (start 118.8346 66.9296) (end 118.8346 66.9236) (width 0.2) (layer "B.Cu") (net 15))
 (segment (start 127.1396 76.2486) (end 127.1396 77.5486) (width 0.2) (layer "F.Cu") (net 18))
 (segment (start 127.1396 77.5486) (end 127.1896 77.5986) (width 0.2) (layer "F.Cu") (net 18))
 (segment (start 127.1896 78.2798) (end 127.1896 77.5986) (width 0.25) (layer "F.Cu") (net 18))
 (via (at 127.1396 76.2486) (size 0.5) (drill 0.3) (layers "F.Cu" "B.Cu") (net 18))
 (segment (start 128.989 66.9244) (end 128.989 66.9246) (width 0.25) (layer "B.Cu") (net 18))
 (segment (start 127.1396 76.2486) (end 127.1396 68.7786) (width 0.2) (layer "B.Cu") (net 18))
 (segment (start 127.1396 68.7786) (end 128.1969 67.7216) (width 0.2) (layer "B.Cu") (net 18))
 (segment (start 128.1969 67.7216) (end 128.9946 66.9236) (width 0.2) (layer "B.Cu") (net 18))
 (segment (start 127.9896 78.2798) (end 127.9896 77.5986) (width 0.25) (layer "F.Cu") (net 19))
 (segment (start 127.9896 75.9236) (end 127.9896 77.5986) (width 0.2) (layer "F.Cu") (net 19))
 (segment (start 128.0146 75.8986) (end 127.9896 75.9236) (width 0.2) (layer "F.Cu") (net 19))
 (via (at 128.0146 75.8986) (size 0.5) (drill 0.3) (layers "F.Cu" "B.Cu") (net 19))
 (segment (start 128.0146 75.8986) (end 128.0146 70.4436) (width 0.2) (layer "B.Cu") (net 19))
 (segment (start 128.0146 70.4436) (end 130.7369 67.7216) (width 0.2) (layer "B.Cu") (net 19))
 (segment (start 130.7369 67.7216) (end 131.5346 66.9236) (width 0.2) (layer "B.Cu") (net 19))
 (segment (start 131.529 66.9244) (end 131.529 66.9246) (width 0.25) (layer "B.Cu") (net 19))
 (segment (start 130.7416 76.8298) (end 129.4396 76.8298) (width 0.2) (layer "F.Cu") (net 20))
 (via (at 130.7416 76.8298) (size 0.5) (drill 0.3) (layers "F.Cu" "B.Cu") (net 20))
 (segment (start 134.069 66.9244) (end 134.069 66.9246) (width 0.25) (layer "B.Cu") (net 20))
 (segment (start 134.0746 66.9236) (end 133.2769 67.7216) (width 0.2) (layer "B.Cu") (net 20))
 (segment (start 130.7416 76.8298) (end 130.7396 76.8278) (width 0.2) (layer "B.Cu") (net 20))
 (segment (start 130.7396 76.8278) (end 130.7396 70.2586) (width 0.2) (layer "B.Cu") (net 20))
 (segment (start 130.7396 70.2586) (end 133.2769 67.7216) (width 0.2) (layer "B.Cu") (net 20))
 (segment (start 129.4521 76.0426) (end 129.4521 76.0423) (width 0.25) (layer "F.Cu") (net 21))
 (segment (start 129.4521 76.1611) (end 129.4521 76.0426) (width 0.25) (layer "F.Cu") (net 21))
 (segment (start 129.4646 76.1736) (end 129.4521 76.1611) (width 0.2) (layer "F.Cu") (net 21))
 (segment (start 129.4521 76.1611) (end 129.4396 76.1486) (width 0.2) (layer "F.Cu") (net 21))
 (segment (start 129.4521 76.0423) (end 129.4396 76.0298) (width 0.25) (layer "F.Cu") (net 21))
 (segment (start 131.3898 76.0298) (end 129.4396 76.0298) (width 0.25) (layer "F.Cu") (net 21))
 (segment (start 131.402 76.0176) (end 131.3898 76.0298) (width 0.25) (layer "F.Cu") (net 21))
 (via (at 131.402 76.0176) (size 0.5) (drill 0.3) (layers "F.Cu" "B.Cu") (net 21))
 (segment (start 131.402 72.1366) (end 135.8169 67.7216) (width 0.2) (layer "B.Cu") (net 21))
 (segment (start 131.402 76.0176) (end 131.402 72.1366) (width 0.2) (layer "B.Cu") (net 21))
 (segment (start 136.6146 66.9236) (end 135.8169 67.7216) (width 0.2) (layer "B.Cu") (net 21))
 (segment (start 136.609 66.9244) (end 136.609 66.9246) (width 0.25) (layer "B.Cu") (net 21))
 (segment (start 129.4396 75.2298) (end 132.5442 75.2298) (width 0.2) (layer "F.Cu") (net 22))
 (segment (start 132.5442 75.2298) (end 132.545 75.2306) (width 0.2) (layer "F.Cu") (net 22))
 (via (at 132.545 75.2306) (size 0.5) (drill 0.3) (layers "F.Cu" "B.Cu") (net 22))
 (segment (start 132.545 73.5336) (end 138.3569 67.7216) (width 0.2) (layer "B.Cu") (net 22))
 (segment (start 132.545 75.2306) (end 132.545 73.5336) (width 0.2) (layer "B.Cu") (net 22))
 (segment (start 139.149 66.9244) (end 139.149 66.9246) (width 0.25) (layer "B.Cu") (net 22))
 (segment (start 138.3569 67.7216) (end 139.1546 66.9236) (width 0.2) (layer "B.Cu") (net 22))
 (segment (start 141.1584 67.4596) (end 141.6946 66.9236) (width 0.2) (layer "F.Cu") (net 23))
 (segment (start 141.6889 66.9244) (end 141.689 66.9244) (width 0.25) (layer "F.Cu") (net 23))
 (segment (start 134.1836 74.4298) (end 141.689 66.9244) (width 0.2) (layer "F.Cu") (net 23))
 (segment (start 141.4237 67.1896) (end 141.689 66.9246) (width 0.25) (layer "F.Cu") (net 23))
 (segment (start 141.4237 67.1896) (end 141.6889 66.9244) (width 0.25) (layer "F.Cu") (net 23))
 (segment (start 129.4396 74.4298) (end 134.1836 74.4298) (width 0.2) (layer "F.Cu") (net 23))
 (segment (start 141.1584 67.4596) (end 141.1584 67.4546) (width 0.25) (layer "F.Cu") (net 23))
 (segment (start 141.1584 67.4546) (end 141.4237 67.1896) (width 0.25) (layer "F.Cu") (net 23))
 (segment (start 134.374 73.6298) (end 140.419 67.5848) (width 0.2) (layer "F.Cu") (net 24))
 (segment (start 141.689 59.3046) (end 141.6877 59.3031) (width 0.25) (layer "F.Cu") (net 24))
 (segment (start 129.4396 73.6298) (end 134.374 73.6298) (width 0.2) (layer "F.Cu") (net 24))
 (segment (start 141.6864 59.3016) (end 141.6896 59.2986) (width 0.2) (layer "F.Cu") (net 24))
 (segment (start 140.419 60.5744) (end 141.689 59.3044) (width 0.2) (layer "F.Cu") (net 24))
 (segment (start 141.6877 59.3031) (end 141.6864 59.3016) (width 0.25) (layer "F.Cu") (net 24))
 (segment (start 141.6877 59.3031) (end 141.689 59.3044) (width 0.25) (layer "F.Cu") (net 24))
 (segment (start 140.419 67.5848) (end 140.419 60.5744) (width 0.2) (layer "F.Cu") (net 24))
 (segment (start 137.879 67.5848) (end 137.879 60.5744) (width 0.2) (layer "F.Cu") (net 25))
 (segment (start 139.149 59.3046) (end 139.1477 59.3031) (width 0.25) (layer "F.Cu") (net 25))
 (segment (start 132.634 72.8298) (end 137.879 67.5848) (width 0.2) (layer "F.Cu") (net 25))
 (segment (start 139.1464 59.3016) (end 139.1496 59.2986) (width 0.2) (layer "F.Cu") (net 25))
 (segment (start 139.1477 59.3031) (end 139.149 59.3044) (width 0.25) (layer "F.Cu") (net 25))
 (segment (start 139.1477 59.3031) (end 139.1464 59.3016) (width 0.25) (layer "F.Cu") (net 25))
 (segment (start 129.4396 72.8298) (end 132.634 72.8298) (width 0.2) (layer "F.Cu") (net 25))
 (segment (start 137.879 60.5744) (end 139.149 59.3044) (width 0.2) (layer "F.Cu") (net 25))
 (segment (start 135.339 60.5744) (end 136.609 59.3044) (width 0.2) (layer "F.Cu") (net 26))
 (segment (start 129.4396 72.0298) (end 130.894 72.0298) (width 0.2) (layer "F.Cu") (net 26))
 (segment (start 130.894 72.0298) (end 135.339 67.5848) (width 0.2) (layer "F.Cu") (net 26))
 (segment (start 136.6077 59.3031) (end 136.609 59.3044) (width 0.25) (layer "F.Cu") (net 26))
 (segment (start 136.6064 59.3016) (end 136.6096 59.2986) (width 0.2) (layer "F.Cu") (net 26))
 (segment (start 136.609 59.3046) (end 136.6077 59.3031) (width 0.25) (layer "F.Cu") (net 26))
 (segment (start 135.339 67.5848) (end 135.339 60.5744) (width 0.2) (layer "F.Cu") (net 26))
 (segment (start 136.6077 59.3031) (end 136.6064 59.3016) (width 0.25) (layer "F.Cu") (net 26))
 (segment (start 129.9414 71.2298) (end 132.8021 68.3691) (width 0.2) (layer "F.Cu") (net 27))
 (segment (start 134.0664 59.3016) (end 134.0696 59.2986) (width 0.2) (layer "F.Cu") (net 27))
 (segment (start 132.8021 60.5656) (end 134.0664 59.3016) (width 0.2) (layer "F.Cu") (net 27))
 (segment (start 134.0677 59.3031) (end 134.069 59.3044) (width 0.25) (layer "F.Cu") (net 27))
 (segment (start 132.8021 68.3691) (end 132.8021 60.5656) (width 0.2) (layer "F.Cu") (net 27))
 (segment (start 134.0677 59.3031) (end 134.0664 59.3016) (width 0.25) (layer "F.Cu") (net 27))
 (segment (start 129.4396 71.2298) (end 129.9414 71.2298) (width 0.2) (layer "F.Cu") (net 27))
 (segment (start 134.069 59.3046) (end 134.0677 59.3031) (width 0.25) (layer "F.Cu") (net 27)))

